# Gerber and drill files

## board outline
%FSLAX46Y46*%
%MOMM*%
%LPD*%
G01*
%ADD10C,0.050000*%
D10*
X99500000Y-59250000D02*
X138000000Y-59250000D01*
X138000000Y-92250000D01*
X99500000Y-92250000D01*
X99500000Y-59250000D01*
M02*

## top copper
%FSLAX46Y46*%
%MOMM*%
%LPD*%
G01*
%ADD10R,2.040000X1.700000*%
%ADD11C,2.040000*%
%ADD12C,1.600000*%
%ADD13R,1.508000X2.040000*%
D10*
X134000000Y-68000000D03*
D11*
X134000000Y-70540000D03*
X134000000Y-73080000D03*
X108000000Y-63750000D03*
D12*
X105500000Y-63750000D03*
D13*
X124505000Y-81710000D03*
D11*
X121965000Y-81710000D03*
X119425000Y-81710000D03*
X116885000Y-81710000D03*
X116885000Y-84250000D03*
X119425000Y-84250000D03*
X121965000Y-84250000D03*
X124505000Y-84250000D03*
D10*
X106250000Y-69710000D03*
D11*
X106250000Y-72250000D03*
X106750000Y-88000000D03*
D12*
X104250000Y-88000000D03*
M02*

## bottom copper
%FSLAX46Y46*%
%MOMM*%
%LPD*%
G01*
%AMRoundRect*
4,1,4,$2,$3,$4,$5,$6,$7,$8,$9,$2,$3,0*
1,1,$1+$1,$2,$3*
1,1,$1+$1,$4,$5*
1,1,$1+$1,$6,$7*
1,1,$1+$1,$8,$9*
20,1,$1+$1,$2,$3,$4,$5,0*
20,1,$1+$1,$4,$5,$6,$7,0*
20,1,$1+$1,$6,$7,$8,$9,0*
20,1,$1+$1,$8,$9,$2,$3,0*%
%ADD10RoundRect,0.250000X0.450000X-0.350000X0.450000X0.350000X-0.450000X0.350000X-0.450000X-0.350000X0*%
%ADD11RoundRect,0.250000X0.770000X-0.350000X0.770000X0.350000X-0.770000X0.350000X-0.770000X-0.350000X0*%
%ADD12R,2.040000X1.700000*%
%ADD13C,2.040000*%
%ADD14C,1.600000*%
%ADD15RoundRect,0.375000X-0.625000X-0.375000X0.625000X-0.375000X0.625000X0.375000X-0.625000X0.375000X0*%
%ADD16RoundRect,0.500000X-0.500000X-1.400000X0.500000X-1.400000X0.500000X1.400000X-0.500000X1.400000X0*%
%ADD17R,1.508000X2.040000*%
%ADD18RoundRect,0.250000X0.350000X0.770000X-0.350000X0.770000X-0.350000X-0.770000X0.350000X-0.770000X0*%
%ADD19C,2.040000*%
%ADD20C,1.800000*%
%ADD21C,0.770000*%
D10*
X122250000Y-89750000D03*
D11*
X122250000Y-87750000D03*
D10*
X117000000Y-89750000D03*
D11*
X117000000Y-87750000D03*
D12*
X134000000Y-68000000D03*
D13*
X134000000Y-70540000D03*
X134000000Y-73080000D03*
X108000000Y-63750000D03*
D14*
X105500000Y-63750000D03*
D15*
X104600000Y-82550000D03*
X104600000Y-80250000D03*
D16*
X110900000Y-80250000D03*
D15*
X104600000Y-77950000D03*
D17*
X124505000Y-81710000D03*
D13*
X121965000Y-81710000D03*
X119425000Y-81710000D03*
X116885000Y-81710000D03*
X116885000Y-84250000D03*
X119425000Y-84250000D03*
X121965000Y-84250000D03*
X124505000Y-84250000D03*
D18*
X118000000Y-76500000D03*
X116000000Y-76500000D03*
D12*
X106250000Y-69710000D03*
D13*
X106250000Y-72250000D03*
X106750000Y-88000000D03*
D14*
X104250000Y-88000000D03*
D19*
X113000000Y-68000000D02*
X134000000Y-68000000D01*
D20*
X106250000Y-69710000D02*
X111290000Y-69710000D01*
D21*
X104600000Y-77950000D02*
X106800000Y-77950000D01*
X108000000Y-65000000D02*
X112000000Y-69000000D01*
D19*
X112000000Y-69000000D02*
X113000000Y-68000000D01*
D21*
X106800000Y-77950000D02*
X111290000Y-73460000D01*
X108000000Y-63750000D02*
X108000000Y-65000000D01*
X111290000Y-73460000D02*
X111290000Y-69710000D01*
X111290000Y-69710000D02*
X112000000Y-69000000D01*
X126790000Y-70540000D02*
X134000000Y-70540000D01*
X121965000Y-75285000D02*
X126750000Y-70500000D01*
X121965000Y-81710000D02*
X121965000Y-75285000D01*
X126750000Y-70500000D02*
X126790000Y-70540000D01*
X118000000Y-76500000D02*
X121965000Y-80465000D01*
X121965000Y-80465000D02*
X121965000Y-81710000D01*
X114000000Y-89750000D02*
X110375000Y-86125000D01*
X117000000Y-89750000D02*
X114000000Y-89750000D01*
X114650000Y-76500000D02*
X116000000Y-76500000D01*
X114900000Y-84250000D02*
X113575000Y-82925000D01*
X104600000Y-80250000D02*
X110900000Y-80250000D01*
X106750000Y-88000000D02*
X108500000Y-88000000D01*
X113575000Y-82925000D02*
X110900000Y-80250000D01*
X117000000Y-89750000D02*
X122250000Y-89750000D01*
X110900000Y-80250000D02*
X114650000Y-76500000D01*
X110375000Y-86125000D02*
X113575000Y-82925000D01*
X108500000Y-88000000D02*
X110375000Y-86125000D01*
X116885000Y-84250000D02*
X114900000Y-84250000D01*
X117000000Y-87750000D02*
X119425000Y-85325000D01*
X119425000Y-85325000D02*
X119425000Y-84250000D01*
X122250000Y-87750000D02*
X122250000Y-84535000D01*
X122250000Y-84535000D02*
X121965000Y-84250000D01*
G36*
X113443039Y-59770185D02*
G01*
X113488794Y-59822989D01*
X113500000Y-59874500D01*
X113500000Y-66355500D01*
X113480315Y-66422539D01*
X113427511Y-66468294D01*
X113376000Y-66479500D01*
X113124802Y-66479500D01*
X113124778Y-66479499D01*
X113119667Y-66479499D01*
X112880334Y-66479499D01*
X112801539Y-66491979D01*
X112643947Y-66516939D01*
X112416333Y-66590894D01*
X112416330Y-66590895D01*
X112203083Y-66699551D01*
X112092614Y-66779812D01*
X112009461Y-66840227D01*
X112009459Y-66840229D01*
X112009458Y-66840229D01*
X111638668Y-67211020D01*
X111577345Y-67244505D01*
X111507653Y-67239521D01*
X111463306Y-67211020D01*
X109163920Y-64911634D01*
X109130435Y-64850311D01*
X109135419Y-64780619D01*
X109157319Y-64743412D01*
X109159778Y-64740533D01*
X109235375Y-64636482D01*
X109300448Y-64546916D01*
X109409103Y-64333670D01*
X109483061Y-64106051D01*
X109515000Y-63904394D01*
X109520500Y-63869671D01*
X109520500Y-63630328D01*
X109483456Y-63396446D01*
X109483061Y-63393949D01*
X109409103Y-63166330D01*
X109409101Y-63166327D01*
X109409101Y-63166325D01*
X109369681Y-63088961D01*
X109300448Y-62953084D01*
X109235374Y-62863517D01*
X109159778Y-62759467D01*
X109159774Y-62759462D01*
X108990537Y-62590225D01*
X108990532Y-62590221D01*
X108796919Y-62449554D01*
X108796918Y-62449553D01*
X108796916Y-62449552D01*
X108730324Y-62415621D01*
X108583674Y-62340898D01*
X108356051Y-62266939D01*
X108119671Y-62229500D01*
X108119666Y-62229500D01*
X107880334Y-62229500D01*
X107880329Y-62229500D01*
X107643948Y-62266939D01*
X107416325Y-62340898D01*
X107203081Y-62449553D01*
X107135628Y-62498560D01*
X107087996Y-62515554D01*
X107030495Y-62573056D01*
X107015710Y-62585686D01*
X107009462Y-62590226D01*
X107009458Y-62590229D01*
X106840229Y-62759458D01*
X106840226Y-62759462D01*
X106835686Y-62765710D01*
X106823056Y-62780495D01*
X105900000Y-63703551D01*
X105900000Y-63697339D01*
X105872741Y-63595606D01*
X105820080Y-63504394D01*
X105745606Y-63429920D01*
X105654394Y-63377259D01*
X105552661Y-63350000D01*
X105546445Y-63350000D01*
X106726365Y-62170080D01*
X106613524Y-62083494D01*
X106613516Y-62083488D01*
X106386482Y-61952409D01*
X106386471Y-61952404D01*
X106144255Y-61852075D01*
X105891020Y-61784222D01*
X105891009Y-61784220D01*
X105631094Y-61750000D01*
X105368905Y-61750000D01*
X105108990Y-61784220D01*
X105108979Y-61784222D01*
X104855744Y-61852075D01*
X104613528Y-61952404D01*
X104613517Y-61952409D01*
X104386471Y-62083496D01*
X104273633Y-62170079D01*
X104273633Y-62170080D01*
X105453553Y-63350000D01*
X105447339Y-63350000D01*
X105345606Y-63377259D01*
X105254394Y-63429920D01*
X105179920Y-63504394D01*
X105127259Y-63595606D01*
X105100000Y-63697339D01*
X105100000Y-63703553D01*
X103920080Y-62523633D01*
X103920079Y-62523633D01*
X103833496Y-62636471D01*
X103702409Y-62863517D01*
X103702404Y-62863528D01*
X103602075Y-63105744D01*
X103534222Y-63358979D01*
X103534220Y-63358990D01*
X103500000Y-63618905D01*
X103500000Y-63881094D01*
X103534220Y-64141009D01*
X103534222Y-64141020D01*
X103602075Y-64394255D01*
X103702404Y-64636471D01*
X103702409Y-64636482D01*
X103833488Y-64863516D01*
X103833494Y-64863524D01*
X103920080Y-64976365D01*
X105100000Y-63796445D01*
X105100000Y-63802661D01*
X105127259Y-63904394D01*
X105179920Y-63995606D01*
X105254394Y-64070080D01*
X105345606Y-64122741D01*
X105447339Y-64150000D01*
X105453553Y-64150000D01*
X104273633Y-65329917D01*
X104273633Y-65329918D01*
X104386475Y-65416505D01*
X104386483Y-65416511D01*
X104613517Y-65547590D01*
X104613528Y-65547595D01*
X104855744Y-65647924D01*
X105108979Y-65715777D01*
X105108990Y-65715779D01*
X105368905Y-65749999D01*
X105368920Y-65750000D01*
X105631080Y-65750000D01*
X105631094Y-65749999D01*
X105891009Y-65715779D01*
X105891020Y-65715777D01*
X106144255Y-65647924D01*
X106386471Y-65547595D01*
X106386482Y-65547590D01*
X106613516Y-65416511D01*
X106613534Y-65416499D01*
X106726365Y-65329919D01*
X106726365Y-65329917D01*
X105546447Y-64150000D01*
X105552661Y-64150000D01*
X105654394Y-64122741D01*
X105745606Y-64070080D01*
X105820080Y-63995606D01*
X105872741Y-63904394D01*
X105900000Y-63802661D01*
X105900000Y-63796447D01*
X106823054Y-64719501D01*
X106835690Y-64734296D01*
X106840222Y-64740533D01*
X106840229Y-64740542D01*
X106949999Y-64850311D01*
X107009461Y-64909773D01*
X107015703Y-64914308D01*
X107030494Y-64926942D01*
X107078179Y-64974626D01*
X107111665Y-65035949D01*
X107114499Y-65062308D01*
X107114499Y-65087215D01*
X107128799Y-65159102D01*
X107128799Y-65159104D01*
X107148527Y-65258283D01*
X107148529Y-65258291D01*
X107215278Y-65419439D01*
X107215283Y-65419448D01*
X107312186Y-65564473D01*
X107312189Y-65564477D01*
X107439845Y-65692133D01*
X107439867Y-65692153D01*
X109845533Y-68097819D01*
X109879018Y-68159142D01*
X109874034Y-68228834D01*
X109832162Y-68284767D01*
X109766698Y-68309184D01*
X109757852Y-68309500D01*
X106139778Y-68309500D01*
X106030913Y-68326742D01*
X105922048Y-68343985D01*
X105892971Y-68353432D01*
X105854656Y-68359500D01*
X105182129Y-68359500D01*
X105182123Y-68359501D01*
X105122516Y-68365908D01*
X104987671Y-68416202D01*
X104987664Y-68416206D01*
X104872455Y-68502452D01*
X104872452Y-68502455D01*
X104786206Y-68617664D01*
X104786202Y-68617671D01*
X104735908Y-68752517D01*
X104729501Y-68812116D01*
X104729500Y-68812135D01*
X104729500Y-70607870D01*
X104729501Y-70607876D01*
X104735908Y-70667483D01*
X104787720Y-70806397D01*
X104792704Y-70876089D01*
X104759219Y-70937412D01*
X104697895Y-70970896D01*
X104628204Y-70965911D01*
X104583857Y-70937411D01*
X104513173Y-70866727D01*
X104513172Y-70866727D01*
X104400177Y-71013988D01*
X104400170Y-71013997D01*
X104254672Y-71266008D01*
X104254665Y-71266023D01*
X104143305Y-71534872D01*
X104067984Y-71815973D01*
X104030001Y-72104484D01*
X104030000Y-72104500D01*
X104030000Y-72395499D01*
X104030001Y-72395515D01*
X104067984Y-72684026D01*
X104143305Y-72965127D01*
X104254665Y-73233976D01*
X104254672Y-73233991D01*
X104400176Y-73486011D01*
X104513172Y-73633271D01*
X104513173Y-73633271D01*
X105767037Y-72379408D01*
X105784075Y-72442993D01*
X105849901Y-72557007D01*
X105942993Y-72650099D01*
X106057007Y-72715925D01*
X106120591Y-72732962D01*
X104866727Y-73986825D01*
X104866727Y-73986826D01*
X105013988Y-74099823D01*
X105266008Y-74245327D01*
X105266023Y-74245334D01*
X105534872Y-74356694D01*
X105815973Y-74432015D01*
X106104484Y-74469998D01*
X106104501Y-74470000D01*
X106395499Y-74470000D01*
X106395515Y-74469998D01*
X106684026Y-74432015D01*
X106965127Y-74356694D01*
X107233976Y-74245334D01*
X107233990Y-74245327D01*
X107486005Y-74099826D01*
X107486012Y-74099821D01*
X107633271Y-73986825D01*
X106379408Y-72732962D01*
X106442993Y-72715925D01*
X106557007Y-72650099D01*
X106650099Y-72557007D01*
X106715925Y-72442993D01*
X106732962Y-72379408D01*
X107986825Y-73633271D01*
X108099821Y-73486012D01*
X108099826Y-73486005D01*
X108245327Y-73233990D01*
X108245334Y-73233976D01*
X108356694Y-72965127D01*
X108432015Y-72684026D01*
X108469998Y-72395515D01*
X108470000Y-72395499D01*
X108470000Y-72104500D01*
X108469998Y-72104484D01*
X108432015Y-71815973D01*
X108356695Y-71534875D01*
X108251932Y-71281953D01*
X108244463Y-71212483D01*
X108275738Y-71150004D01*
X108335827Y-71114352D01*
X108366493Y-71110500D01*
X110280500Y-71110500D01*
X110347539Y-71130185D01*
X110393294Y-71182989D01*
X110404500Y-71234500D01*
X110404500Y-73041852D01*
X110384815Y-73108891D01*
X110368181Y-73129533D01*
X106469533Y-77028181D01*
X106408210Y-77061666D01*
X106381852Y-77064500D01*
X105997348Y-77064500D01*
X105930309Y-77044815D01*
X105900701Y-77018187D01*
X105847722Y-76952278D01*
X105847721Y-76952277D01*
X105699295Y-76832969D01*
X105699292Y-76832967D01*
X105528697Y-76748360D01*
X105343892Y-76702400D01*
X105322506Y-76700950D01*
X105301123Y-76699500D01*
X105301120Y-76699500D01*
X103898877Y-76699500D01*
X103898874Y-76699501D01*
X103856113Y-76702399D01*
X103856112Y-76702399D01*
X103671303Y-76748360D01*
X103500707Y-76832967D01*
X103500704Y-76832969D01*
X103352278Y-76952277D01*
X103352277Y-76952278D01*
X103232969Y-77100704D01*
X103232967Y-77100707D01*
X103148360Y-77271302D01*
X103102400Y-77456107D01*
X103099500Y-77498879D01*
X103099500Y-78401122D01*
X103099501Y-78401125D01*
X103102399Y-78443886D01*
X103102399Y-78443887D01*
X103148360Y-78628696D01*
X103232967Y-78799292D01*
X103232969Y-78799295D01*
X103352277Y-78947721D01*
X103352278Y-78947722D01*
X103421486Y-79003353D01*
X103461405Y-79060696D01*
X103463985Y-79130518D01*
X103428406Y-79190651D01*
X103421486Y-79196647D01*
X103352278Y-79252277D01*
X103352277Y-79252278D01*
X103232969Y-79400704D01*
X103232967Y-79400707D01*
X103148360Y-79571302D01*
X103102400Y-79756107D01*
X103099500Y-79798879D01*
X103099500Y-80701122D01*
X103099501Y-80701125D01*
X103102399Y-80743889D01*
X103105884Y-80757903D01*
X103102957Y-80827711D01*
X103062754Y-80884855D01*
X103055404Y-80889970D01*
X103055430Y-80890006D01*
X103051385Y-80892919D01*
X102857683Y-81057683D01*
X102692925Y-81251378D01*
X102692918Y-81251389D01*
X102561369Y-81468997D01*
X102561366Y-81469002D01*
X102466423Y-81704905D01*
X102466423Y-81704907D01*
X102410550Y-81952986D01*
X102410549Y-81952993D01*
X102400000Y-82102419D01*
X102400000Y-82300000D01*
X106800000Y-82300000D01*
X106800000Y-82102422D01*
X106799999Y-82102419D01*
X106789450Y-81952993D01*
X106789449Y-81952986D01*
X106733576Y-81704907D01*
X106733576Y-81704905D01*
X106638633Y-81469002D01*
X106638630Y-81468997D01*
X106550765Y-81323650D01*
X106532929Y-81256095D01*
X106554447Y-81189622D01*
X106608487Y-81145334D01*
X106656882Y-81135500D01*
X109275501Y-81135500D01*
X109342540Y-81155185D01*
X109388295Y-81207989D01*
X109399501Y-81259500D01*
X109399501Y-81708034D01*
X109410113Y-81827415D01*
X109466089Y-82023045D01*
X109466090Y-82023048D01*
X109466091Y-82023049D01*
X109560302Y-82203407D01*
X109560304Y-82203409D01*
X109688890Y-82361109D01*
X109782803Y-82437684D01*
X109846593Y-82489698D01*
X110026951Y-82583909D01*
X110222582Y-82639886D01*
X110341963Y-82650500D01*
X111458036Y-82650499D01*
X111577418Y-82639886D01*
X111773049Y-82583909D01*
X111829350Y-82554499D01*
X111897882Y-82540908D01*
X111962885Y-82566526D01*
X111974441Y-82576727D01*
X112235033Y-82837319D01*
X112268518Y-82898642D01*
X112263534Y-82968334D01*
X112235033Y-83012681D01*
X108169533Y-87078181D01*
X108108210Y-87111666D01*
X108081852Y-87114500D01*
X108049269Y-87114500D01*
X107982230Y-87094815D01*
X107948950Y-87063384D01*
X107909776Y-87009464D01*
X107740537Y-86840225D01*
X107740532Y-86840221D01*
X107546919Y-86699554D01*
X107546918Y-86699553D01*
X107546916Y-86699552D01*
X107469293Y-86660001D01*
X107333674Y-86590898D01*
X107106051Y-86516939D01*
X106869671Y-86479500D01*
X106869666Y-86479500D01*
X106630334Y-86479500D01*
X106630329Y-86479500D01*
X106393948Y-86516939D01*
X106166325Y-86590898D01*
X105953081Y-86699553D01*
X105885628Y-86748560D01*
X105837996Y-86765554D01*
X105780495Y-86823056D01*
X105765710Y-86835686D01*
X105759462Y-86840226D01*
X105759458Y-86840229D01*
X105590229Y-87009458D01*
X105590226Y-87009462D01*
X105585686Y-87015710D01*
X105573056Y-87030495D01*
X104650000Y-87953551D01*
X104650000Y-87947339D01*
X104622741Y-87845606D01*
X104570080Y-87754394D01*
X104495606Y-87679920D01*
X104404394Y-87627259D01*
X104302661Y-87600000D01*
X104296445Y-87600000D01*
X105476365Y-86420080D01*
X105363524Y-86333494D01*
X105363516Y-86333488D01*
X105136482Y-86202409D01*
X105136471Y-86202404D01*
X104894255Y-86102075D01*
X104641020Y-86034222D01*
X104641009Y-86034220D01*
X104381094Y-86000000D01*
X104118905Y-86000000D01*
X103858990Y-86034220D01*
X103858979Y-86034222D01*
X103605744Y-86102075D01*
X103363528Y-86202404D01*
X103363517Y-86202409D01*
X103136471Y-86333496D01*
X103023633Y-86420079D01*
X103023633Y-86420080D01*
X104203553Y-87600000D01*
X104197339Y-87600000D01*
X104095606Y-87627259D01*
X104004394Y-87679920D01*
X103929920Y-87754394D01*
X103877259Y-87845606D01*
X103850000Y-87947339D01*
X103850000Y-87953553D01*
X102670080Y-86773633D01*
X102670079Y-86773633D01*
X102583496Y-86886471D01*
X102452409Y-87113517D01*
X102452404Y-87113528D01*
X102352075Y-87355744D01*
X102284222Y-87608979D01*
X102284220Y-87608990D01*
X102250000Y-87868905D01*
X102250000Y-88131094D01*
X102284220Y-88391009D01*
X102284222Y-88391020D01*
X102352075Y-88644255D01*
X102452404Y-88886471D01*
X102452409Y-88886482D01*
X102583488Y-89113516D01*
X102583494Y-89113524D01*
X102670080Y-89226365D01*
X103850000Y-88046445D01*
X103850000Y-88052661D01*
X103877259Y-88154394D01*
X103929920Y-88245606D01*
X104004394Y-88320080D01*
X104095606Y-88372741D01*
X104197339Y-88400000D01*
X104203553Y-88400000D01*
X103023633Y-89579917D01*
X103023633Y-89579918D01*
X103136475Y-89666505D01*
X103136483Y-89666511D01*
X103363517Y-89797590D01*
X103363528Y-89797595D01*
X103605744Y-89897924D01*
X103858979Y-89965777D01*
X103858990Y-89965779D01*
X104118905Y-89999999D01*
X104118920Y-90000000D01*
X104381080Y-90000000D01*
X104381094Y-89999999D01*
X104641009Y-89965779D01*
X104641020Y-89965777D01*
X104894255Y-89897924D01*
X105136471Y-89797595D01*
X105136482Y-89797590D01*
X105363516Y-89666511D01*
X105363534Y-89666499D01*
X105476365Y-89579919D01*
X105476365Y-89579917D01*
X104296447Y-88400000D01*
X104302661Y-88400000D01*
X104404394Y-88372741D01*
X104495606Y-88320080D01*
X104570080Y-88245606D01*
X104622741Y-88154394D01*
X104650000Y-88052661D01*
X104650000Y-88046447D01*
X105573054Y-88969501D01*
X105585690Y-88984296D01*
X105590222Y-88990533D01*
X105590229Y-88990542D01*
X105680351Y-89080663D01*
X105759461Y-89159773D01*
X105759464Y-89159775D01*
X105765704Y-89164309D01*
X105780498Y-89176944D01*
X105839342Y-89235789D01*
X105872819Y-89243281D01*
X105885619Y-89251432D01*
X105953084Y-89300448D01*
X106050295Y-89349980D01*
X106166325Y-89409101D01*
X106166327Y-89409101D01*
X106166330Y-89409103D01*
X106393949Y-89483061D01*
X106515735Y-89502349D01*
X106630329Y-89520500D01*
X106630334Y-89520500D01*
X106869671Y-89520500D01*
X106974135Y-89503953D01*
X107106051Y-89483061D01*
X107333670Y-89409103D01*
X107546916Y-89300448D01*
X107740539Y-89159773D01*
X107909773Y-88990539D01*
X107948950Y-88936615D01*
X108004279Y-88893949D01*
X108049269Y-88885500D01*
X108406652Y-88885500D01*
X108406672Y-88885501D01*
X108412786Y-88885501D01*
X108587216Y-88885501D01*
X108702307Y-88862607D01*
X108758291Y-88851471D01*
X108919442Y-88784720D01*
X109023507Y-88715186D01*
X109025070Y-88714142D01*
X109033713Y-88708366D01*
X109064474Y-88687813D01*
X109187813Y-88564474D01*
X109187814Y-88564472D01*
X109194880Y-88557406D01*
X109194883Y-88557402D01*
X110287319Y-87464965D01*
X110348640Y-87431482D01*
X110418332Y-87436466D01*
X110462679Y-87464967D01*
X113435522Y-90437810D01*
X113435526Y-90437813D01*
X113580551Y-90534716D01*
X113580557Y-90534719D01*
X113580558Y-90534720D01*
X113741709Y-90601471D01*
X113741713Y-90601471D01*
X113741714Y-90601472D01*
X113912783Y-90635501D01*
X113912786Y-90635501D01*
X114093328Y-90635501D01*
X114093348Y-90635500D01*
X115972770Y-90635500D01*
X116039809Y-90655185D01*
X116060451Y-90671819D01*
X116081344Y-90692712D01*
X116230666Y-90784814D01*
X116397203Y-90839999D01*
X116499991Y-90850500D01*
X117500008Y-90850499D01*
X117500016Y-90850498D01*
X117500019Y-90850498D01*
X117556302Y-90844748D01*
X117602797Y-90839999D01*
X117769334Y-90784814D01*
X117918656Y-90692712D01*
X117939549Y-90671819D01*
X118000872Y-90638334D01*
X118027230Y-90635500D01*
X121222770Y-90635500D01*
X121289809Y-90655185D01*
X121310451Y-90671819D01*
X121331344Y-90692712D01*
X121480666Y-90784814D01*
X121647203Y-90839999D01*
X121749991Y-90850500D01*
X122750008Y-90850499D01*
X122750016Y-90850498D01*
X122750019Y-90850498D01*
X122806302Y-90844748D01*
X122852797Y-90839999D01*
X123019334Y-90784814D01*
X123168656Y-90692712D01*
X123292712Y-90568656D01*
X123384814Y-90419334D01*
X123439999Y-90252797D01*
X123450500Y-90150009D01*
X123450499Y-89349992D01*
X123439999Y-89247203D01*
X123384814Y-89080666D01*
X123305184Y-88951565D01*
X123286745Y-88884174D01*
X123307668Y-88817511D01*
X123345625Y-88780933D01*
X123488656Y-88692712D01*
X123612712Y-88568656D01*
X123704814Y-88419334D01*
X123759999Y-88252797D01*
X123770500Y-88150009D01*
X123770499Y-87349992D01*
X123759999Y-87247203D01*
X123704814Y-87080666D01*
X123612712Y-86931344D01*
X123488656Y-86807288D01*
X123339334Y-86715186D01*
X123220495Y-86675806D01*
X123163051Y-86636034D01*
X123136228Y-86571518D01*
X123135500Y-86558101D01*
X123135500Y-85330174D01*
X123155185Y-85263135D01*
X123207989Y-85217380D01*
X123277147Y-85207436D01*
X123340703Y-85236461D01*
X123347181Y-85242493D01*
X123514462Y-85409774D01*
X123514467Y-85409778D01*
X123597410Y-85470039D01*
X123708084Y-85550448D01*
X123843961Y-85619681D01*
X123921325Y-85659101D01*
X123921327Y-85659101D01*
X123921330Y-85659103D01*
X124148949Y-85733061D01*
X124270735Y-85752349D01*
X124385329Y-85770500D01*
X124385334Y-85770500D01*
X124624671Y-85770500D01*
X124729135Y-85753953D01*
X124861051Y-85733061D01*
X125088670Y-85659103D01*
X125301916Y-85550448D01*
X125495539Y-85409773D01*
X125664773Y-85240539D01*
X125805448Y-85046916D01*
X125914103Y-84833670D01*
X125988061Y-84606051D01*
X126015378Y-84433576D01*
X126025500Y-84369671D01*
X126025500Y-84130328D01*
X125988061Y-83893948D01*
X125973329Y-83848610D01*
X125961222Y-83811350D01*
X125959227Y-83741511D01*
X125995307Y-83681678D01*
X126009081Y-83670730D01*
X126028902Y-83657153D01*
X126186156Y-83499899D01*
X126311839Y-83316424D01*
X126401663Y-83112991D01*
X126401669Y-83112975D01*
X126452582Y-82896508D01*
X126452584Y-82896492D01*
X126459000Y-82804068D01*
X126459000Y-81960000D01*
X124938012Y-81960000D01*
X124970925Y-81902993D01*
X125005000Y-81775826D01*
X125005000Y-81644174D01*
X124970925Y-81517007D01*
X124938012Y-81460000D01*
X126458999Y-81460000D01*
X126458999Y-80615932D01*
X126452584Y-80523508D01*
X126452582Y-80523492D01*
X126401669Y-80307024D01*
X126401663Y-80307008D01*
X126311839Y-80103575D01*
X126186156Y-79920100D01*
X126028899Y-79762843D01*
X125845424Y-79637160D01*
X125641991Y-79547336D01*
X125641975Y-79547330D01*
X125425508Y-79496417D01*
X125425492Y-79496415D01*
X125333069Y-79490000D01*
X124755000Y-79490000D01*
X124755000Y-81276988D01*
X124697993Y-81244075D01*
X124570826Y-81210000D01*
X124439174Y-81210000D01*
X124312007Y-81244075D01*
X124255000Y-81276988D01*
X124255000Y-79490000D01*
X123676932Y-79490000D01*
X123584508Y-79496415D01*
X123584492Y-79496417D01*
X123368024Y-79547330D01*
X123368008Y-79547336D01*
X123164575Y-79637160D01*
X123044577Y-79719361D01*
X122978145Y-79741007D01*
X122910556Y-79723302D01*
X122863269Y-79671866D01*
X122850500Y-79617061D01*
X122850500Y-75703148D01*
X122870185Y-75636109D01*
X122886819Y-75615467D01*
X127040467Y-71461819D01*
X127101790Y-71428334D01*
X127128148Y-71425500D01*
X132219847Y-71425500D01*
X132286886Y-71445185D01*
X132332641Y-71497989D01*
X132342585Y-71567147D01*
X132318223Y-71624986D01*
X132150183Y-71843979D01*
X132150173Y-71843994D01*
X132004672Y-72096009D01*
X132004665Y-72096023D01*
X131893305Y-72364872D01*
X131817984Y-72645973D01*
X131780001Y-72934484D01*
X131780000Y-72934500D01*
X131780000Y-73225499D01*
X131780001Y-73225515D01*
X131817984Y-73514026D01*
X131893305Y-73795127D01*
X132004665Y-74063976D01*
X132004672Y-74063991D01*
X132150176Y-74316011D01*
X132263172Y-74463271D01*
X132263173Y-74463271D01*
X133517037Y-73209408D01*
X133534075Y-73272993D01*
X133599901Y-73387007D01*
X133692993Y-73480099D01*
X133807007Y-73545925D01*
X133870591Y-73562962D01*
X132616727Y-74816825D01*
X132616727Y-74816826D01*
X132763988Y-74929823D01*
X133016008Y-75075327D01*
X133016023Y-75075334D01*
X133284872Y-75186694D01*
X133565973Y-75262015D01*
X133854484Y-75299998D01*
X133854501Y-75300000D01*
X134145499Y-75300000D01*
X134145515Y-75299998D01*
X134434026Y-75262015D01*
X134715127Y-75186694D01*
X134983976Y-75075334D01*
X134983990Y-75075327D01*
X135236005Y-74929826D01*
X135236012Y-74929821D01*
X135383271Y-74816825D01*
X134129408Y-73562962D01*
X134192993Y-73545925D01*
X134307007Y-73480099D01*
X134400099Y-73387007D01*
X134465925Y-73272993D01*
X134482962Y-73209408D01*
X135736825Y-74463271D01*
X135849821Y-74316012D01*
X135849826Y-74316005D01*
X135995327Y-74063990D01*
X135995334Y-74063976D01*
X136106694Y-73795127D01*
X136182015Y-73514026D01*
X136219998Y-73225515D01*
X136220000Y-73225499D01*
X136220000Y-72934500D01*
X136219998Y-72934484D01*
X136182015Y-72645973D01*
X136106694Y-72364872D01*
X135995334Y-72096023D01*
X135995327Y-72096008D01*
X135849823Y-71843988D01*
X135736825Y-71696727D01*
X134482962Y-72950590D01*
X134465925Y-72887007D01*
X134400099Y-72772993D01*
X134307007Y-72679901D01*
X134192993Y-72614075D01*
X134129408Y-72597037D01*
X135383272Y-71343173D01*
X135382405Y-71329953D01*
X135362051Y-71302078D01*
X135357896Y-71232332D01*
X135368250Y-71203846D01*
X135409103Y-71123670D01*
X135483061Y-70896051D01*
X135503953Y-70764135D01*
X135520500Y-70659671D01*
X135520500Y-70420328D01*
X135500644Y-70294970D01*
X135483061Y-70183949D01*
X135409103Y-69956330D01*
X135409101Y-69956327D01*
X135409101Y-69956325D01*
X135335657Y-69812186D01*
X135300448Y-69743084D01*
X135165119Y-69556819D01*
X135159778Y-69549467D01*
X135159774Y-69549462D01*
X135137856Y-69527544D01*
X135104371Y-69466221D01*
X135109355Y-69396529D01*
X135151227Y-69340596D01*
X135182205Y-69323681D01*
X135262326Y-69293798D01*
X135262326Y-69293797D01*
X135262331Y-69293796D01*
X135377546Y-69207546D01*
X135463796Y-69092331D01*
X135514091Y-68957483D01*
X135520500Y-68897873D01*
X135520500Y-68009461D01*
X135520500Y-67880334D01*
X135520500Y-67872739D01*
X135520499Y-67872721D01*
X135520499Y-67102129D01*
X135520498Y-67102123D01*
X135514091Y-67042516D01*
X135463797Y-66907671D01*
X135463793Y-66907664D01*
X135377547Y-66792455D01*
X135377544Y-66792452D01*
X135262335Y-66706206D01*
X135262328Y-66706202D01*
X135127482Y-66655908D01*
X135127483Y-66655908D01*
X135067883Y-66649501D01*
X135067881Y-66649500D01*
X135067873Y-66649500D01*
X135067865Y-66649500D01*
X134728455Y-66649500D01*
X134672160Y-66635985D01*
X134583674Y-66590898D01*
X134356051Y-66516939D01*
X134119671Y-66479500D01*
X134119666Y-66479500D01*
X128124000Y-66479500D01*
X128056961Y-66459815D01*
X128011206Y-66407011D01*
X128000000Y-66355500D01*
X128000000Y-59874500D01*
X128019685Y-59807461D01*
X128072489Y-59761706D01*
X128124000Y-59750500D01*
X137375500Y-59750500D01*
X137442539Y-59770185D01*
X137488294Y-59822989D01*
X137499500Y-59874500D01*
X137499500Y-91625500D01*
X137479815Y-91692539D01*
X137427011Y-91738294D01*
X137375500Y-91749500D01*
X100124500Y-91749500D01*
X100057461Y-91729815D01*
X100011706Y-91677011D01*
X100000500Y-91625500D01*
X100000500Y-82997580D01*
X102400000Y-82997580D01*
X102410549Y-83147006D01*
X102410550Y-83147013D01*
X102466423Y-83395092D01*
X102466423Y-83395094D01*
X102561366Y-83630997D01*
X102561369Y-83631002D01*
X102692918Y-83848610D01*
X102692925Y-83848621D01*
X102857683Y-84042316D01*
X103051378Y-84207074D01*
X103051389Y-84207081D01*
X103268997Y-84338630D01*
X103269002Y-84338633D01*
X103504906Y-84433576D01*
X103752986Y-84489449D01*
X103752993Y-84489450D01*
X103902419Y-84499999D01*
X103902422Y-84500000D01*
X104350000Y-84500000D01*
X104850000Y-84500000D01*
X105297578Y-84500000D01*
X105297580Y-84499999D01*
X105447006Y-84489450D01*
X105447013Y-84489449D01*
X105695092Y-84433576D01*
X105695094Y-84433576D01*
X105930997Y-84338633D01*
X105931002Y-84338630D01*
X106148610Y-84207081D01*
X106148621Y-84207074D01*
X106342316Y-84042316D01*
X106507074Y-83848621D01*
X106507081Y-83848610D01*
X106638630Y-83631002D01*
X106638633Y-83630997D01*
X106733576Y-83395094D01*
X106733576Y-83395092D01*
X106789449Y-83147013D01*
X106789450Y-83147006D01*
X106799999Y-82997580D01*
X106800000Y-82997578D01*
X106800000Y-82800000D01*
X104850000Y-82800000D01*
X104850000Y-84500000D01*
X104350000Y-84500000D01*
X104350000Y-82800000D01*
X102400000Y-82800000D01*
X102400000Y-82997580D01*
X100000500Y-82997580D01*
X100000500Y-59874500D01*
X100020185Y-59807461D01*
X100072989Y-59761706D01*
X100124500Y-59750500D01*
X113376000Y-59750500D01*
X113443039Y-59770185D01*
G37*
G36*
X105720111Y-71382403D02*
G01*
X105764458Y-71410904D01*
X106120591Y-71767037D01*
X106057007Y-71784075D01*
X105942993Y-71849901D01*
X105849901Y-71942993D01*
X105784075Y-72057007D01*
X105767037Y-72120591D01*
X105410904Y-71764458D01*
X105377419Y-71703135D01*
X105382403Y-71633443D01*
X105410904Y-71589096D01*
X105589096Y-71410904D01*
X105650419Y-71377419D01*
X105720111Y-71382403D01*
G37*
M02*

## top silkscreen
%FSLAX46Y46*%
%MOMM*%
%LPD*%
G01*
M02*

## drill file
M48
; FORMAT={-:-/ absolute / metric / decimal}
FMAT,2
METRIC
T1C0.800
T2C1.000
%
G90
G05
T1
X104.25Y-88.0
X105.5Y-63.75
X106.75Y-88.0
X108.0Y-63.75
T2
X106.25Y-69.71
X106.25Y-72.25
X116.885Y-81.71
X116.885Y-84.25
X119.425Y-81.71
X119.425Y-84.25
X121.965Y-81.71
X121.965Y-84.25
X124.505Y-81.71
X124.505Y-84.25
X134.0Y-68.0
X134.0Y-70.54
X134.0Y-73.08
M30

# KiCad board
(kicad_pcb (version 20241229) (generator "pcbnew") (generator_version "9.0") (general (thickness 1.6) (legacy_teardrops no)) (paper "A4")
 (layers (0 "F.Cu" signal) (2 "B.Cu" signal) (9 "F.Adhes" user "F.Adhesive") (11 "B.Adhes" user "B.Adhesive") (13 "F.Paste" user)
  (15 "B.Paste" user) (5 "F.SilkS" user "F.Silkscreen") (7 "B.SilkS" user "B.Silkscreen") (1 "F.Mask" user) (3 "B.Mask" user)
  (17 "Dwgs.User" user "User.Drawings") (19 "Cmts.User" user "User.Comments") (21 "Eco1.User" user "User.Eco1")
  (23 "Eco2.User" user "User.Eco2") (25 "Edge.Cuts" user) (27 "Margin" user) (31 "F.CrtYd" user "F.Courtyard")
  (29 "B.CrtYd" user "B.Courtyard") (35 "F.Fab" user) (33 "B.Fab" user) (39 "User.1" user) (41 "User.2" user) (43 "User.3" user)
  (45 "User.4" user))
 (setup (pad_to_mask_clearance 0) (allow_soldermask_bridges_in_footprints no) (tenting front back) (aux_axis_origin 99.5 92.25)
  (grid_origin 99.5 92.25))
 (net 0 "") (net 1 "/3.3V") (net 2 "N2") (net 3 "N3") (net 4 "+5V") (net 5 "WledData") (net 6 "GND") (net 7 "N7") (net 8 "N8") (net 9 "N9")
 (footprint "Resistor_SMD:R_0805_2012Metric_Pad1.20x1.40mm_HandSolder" (layer "B.Cu") (at 122.25 88.75 90)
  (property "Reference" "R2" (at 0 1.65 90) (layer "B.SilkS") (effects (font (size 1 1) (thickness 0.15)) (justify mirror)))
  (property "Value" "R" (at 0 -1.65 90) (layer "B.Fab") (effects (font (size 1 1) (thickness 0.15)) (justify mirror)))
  (pad "1" smd roundrect (at -1 0 90) (size 1.2 1.4) (layers "B.Cu" "B.Mask" "B.Paste") (roundrect_rratio 0.208333) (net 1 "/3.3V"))
  (pad "2" smd roundrect (at 1 0 90) (size 1.2 2.04) (layers "B.Cu" "B.Mask" "B.Paste") (roundrect_rratio 0.208333) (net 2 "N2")))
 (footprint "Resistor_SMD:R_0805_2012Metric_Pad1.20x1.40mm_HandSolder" (layer "B.Cu") (at 117 88.75 90)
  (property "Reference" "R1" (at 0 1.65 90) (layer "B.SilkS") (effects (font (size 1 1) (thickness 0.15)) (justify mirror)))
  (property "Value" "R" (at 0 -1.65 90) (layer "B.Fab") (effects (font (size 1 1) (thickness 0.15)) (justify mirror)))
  (pad "1" smd roundrect (at -1 0 90) (size 1.2 1.4) (layers "B.Cu" "B.Mask" "B.Paste") (roundrect_rratio 0.208333) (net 1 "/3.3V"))
  (pad "2" smd roundrect (at 1 0 90) (size 1.2 2.04) (layers "B.Cu" "B.Mask" "B.Paste") (roundrect_rratio 0.208333) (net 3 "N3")))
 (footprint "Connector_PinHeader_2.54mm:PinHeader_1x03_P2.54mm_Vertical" (layer "B.Cu") (at 134 68 180)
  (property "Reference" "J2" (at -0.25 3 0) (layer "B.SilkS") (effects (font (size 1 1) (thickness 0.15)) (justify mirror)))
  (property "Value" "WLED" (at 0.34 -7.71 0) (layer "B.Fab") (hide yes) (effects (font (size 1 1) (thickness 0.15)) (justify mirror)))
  (pad "1" thru_hole rect (at 0 0 180) (size 2.04 1.7) (drill 1) (layers "*.Cu" "*.Mask") (remove_unused_layers no) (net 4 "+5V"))
  (pad "2" thru_hole circle (at 0 -2.54 180) (size 2.04 2.04) (drill 1) (layers "*.Cu" "*.Mask") (remove_unused_layers no)
   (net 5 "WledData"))
  (pad "3" thru_hole circle (at 0 -5.08 180) (size 2.04 2.04) (drill 1) (layers "*.Cu" "*.Mask") (remove_unused_layers no) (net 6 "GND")))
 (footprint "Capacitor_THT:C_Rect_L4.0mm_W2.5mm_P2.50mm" (layer "B.Cu") (at 108 63.75 180)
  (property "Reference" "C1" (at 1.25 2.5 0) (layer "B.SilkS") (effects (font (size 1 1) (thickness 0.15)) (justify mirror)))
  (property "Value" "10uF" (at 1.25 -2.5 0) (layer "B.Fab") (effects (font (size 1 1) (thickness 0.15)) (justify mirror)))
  (pad "1" thru_hole circle (at 0 0 180) (size 2.04 2.04) (drill 0.8) (layers "*.Cu" "*.Mask") (remove_unused_layers no) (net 4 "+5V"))
  (pad "2" thru_hole circle (at 2.5 0 180) (size 1.6 1.6) (drill 0.8) (layers "*.Cu" "*.Mask") (remove_unused_layers no) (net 6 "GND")))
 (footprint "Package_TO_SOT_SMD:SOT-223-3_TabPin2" (layer "B.Cu") (at 107.75 80.25)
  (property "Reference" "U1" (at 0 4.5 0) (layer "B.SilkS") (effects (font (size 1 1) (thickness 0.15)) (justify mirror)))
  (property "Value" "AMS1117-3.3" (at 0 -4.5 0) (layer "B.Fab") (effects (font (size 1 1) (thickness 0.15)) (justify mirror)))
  (pad "1" smd roundrect (at -3.15 2.3) (size 2 1.5) (layers "B.Cu" "B.Mask" "B.Paste") (roundrect_rratio 0.25) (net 6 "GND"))
  (pad "2" smd roundrect (at -3.15 0) (size 2 1.5) (layers "B.Cu" "B.Mask" "B.Paste") (roundrect_rratio 0.25) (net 1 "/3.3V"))
  (pad "2" smd roundrect (at 3.15 0) (size 2 3.8) (layers "B.Cu" "B.Mask" "B.Paste") (roundrect_rratio 0.25) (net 1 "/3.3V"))
  (pad "3" smd roundrect (at -3.15 -2.3) (size 2 1.5) (layers "B.Cu" "B.Mask" "B.Paste") (roundrect_rratio 0.25) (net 4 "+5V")))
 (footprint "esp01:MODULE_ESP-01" (layer "B.Cu") (at 120.695 73.35 180)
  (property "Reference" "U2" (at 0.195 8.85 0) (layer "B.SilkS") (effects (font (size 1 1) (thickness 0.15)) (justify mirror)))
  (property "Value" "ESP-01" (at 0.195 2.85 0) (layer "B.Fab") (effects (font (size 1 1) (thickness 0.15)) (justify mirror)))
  (pad "1" thru_hole rect (at -3.81 -8.36 180) (size 1.508 2.04) (drill 1) (layers "*.Cu" "*.Mask") (remove_unused_layers no) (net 6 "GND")
   (solder_mask_margin 0.102))
  (pad "2" thru_hole circle (at -1.27 -8.36 180) (size 2.04 2.04) (drill 1) (layers "*.Cu" "*.Mask") (remove_unused_layers no)
   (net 5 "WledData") (solder_mask_margin 0.102))
  (pad "3" thru_hole circle (at 1.27 -8.36 180) (size 2.04 2.04) (drill 1) (layers "*.Cu" "*.Mask") (remove_unused_layers no) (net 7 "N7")
   (solder_mask_margin 0.102))
  (pad "4" thru_hole circle (at 3.81 -8.36 180) (size 2.04 2.04) (drill 1) (layers "*.Cu" "*.Mask") (remove_unused_layers no) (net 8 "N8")
   (solder_mask_margin 0.102))
  (pad "5" thru_hole circle (at 3.81 -10.9 180) (size 2.04 2.04) (drill 1) (layers "*.Cu" "*.Mask") (remove_unused_layers no)
   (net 1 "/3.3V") (solder_mask_margin 0.102))
  (pad "6" thru_hole circle (at 1.27 -10.9 180) (size 2.04 2.04) (drill 1) (layers "*.Cu" "*.Mask") (remove_unused_layers no) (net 3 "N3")
   (solder_mask_margin 0.102))
  (pad "7" thru_hole circle (at -1.27 -10.9 180) (size 2.04 2.04) (drill 1) (layers "*.Cu" "*.Mask") (remove_unused_layers no) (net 2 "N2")
   (solder_mask_margin 0.102))
  (pad "8" thru_hole circle (at -3.81 -10.9 180) (size 2.04 2.04) (drill 1) (layers "*.Cu" "*.Mask") (remove_unused_layers no) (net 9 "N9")
   (solder_mask_margin 0.102)))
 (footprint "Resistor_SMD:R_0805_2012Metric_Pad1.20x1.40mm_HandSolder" (layer "B.Cu") (at 117 76.5 180)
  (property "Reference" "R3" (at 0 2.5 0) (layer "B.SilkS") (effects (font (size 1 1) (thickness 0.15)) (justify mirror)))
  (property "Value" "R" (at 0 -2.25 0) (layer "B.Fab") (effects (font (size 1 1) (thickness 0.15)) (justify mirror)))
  (pad "1" smd roundrect (at -1 0 180) (size 1.2 2.04) (layers "B.Cu" "B.Mask" "B.Paste") (roundrect_rratio 0.208333) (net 5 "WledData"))
  (pad "2" smd roundrect (at 1 0 180) (size 1.2 2.04) (layers "B.Cu" "B.Mask" "B.Paste") (roundrect_rratio 0.208333) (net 1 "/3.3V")))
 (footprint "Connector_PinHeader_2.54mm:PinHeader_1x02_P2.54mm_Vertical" (layer "B.Cu") (at 106.25 69.71 180)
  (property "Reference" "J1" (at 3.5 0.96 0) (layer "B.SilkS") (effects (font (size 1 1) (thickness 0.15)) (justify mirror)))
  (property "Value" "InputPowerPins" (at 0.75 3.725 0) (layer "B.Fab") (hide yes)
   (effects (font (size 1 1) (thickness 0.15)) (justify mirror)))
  (pad "1" thru_hole rect (at 0 0 180) (size 2.04 1.7) (drill 1) (layers "*.Cu" "*.Mask") (remove_unused_layers no) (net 4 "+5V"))
  (pad "2" thru_hole circle (at 0 -2.54 180) (size 2.04 2.04) (drill 1) (layers "*.Cu" "*.Mask") (remove_unused_layers no) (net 6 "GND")))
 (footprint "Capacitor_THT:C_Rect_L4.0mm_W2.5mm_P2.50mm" (layer "B.Cu") (at 106.75 88 180)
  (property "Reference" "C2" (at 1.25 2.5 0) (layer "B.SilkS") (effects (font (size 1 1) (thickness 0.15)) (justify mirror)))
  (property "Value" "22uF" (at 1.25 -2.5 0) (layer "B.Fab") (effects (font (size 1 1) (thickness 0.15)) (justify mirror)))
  (pad "1" thru_hole circle (at 0 0 180) (size 2.04 2.04) (drill 0.8) (layers "*.Cu" "*.Mask") (remove_unused_layers no) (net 1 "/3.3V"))
  (pad "2" thru_hole circle (at 2.5 0 180) (size 1.6 1.6) (drill 0.8) (layers "*.Cu" "*.Mask") (remove_unused_layers no) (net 6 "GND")))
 (gr_rect (start 99.5 59.25) (end 138 92.25) (stroke (width 0.05) (type default)) (fill no) (layer "Edge.Cuts"))
 (segment (start 113 68) (end 134 68) (width 2.04) (layer "B.Cu") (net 4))
 (segment (start 106.25 69.71) (end 111.29 69.71) (width 1.8) (layer "B.Cu") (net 4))
 (segment (start 104.6 77.95) (end 106.8 77.95) (width 0.77) (layer "B.Cu") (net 4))
 (segment (start 108 65) (end 112 69) (width 0.77) (layer "B.Cu") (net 4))
 (segment (start 112 69) (end 113 68) (width 2.04) (layer "B.Cu") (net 4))
 (segment (start 106.8 77.95) (end 111.29 73.46) (width 0.77) (layer "B.Cu") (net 4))
 (segment (start 108 63.75) (end 108 65) (width 0.77) (layer "B.Cu") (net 4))
 (segment (start 111.29 73.46) (end 111.29 69.71) (width 0.77) (layer "B.Cu") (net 4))
 (segment (start 111.29 69.71) (end 112 69) (width 0.77) (layer "B.Cu") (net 4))
 (segment (start 126.79 70.54) (end 134 70.54) (width 0.77) (layer "B.Cu") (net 5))
 (segment (start 121.965 75.285) (end 126.75 70.5) (width 0.77) (layer "B.Cu") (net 5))
 (segment (start 121.965 81.71) (end 121.965 75.285) (width 0.77) (layer "B.Cu") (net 5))
 (segment (start 126.75 70.5) (end 126.79 70.54) (width 0.77) (layer "B.Cu") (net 5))
 (segment (start 118 76.5) (end 121.965 80.465) (width 0.77) (layer "B.Cu") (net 5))
 (segment (start 121.965 80.465) (end 121.965 81.71) (width 0.77) (layer "B.Cu") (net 5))
 (segment (start 114 89.75) (end 110.375 86.125) (width 0.77) (layer "B.Cu") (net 1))
 (segment (start 117 89.75) (end 114 89.75) (width 0.77) (layer "B.Cu") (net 1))
 (segment (start 114.65 76.5) (end 116 76.5) (width 0.77) (layer "B.Cu") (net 1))
 (segment (start 114.9 84.25) (end 113.575 82.925) (width 0.77) (layer "B.Cu") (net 1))
 (segment (start 104.6 80.25) (end 110.9 80.25) (width 0.77) (layer "B.Cu") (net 1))
 (segment (start 106.75 88) (end 108.5 88) (width 0.77) (layer "B.Cu") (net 1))
 (segment (start 113.575 82.925) (end 110.9 80.25) (width 0.77) (layer "B.Cu") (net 1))
 (segment (start 117 89.75) (end 122.25 89.75) (width 0.77) (layer "B.Cu") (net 1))
 (segment (start 110.9 80.25) (end 114.65 76.5) (width 0.77) (layer "B.Cu") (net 1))
 (segment (start 110.375 86.125) (end 113.575 82.925) (width 0.77) (layer "B.Cu") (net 1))
 (segment (start 108.5 88) (end 110.375 86.125) (width 0.77) (layer "B.Cu") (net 1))
 (segment (start 116.885 84.25) (end 114.9 84.25) (width 0.77) (layer "B.Cu") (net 1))
 (segment (start 117 87.75) (end 119.425 85.325) (width 0.77) (layer "B.Cu") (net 3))
 (segment (start 119.425 85.325) (end 119.425 84.25) (width 0.77) (layer "B.Cu") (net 3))
 (segment (start 122.25 87.75) (end 122.25 84.535) (width 0.77) (layer "B.Cu") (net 2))
 (segment (start 122.25 84.535) (end 121.965 84.25) (width 0.77) (layer "B.Cu") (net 2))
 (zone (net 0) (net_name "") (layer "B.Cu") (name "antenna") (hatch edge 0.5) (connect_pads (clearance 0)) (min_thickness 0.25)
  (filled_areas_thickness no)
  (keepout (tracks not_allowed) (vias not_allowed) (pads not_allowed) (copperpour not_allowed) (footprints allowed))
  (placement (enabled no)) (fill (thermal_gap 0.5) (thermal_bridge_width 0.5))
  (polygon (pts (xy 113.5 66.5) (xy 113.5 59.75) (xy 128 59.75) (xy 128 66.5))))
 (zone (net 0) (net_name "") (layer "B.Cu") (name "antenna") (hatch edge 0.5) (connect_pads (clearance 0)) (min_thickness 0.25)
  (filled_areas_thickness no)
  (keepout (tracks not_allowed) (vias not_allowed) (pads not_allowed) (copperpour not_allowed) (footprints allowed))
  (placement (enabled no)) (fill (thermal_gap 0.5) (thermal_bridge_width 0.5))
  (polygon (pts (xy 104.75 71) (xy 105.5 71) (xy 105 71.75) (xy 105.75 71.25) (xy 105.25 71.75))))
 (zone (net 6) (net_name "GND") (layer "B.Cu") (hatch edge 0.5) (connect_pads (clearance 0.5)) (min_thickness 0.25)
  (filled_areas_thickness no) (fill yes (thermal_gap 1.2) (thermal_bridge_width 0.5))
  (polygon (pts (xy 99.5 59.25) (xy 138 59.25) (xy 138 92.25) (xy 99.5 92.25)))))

